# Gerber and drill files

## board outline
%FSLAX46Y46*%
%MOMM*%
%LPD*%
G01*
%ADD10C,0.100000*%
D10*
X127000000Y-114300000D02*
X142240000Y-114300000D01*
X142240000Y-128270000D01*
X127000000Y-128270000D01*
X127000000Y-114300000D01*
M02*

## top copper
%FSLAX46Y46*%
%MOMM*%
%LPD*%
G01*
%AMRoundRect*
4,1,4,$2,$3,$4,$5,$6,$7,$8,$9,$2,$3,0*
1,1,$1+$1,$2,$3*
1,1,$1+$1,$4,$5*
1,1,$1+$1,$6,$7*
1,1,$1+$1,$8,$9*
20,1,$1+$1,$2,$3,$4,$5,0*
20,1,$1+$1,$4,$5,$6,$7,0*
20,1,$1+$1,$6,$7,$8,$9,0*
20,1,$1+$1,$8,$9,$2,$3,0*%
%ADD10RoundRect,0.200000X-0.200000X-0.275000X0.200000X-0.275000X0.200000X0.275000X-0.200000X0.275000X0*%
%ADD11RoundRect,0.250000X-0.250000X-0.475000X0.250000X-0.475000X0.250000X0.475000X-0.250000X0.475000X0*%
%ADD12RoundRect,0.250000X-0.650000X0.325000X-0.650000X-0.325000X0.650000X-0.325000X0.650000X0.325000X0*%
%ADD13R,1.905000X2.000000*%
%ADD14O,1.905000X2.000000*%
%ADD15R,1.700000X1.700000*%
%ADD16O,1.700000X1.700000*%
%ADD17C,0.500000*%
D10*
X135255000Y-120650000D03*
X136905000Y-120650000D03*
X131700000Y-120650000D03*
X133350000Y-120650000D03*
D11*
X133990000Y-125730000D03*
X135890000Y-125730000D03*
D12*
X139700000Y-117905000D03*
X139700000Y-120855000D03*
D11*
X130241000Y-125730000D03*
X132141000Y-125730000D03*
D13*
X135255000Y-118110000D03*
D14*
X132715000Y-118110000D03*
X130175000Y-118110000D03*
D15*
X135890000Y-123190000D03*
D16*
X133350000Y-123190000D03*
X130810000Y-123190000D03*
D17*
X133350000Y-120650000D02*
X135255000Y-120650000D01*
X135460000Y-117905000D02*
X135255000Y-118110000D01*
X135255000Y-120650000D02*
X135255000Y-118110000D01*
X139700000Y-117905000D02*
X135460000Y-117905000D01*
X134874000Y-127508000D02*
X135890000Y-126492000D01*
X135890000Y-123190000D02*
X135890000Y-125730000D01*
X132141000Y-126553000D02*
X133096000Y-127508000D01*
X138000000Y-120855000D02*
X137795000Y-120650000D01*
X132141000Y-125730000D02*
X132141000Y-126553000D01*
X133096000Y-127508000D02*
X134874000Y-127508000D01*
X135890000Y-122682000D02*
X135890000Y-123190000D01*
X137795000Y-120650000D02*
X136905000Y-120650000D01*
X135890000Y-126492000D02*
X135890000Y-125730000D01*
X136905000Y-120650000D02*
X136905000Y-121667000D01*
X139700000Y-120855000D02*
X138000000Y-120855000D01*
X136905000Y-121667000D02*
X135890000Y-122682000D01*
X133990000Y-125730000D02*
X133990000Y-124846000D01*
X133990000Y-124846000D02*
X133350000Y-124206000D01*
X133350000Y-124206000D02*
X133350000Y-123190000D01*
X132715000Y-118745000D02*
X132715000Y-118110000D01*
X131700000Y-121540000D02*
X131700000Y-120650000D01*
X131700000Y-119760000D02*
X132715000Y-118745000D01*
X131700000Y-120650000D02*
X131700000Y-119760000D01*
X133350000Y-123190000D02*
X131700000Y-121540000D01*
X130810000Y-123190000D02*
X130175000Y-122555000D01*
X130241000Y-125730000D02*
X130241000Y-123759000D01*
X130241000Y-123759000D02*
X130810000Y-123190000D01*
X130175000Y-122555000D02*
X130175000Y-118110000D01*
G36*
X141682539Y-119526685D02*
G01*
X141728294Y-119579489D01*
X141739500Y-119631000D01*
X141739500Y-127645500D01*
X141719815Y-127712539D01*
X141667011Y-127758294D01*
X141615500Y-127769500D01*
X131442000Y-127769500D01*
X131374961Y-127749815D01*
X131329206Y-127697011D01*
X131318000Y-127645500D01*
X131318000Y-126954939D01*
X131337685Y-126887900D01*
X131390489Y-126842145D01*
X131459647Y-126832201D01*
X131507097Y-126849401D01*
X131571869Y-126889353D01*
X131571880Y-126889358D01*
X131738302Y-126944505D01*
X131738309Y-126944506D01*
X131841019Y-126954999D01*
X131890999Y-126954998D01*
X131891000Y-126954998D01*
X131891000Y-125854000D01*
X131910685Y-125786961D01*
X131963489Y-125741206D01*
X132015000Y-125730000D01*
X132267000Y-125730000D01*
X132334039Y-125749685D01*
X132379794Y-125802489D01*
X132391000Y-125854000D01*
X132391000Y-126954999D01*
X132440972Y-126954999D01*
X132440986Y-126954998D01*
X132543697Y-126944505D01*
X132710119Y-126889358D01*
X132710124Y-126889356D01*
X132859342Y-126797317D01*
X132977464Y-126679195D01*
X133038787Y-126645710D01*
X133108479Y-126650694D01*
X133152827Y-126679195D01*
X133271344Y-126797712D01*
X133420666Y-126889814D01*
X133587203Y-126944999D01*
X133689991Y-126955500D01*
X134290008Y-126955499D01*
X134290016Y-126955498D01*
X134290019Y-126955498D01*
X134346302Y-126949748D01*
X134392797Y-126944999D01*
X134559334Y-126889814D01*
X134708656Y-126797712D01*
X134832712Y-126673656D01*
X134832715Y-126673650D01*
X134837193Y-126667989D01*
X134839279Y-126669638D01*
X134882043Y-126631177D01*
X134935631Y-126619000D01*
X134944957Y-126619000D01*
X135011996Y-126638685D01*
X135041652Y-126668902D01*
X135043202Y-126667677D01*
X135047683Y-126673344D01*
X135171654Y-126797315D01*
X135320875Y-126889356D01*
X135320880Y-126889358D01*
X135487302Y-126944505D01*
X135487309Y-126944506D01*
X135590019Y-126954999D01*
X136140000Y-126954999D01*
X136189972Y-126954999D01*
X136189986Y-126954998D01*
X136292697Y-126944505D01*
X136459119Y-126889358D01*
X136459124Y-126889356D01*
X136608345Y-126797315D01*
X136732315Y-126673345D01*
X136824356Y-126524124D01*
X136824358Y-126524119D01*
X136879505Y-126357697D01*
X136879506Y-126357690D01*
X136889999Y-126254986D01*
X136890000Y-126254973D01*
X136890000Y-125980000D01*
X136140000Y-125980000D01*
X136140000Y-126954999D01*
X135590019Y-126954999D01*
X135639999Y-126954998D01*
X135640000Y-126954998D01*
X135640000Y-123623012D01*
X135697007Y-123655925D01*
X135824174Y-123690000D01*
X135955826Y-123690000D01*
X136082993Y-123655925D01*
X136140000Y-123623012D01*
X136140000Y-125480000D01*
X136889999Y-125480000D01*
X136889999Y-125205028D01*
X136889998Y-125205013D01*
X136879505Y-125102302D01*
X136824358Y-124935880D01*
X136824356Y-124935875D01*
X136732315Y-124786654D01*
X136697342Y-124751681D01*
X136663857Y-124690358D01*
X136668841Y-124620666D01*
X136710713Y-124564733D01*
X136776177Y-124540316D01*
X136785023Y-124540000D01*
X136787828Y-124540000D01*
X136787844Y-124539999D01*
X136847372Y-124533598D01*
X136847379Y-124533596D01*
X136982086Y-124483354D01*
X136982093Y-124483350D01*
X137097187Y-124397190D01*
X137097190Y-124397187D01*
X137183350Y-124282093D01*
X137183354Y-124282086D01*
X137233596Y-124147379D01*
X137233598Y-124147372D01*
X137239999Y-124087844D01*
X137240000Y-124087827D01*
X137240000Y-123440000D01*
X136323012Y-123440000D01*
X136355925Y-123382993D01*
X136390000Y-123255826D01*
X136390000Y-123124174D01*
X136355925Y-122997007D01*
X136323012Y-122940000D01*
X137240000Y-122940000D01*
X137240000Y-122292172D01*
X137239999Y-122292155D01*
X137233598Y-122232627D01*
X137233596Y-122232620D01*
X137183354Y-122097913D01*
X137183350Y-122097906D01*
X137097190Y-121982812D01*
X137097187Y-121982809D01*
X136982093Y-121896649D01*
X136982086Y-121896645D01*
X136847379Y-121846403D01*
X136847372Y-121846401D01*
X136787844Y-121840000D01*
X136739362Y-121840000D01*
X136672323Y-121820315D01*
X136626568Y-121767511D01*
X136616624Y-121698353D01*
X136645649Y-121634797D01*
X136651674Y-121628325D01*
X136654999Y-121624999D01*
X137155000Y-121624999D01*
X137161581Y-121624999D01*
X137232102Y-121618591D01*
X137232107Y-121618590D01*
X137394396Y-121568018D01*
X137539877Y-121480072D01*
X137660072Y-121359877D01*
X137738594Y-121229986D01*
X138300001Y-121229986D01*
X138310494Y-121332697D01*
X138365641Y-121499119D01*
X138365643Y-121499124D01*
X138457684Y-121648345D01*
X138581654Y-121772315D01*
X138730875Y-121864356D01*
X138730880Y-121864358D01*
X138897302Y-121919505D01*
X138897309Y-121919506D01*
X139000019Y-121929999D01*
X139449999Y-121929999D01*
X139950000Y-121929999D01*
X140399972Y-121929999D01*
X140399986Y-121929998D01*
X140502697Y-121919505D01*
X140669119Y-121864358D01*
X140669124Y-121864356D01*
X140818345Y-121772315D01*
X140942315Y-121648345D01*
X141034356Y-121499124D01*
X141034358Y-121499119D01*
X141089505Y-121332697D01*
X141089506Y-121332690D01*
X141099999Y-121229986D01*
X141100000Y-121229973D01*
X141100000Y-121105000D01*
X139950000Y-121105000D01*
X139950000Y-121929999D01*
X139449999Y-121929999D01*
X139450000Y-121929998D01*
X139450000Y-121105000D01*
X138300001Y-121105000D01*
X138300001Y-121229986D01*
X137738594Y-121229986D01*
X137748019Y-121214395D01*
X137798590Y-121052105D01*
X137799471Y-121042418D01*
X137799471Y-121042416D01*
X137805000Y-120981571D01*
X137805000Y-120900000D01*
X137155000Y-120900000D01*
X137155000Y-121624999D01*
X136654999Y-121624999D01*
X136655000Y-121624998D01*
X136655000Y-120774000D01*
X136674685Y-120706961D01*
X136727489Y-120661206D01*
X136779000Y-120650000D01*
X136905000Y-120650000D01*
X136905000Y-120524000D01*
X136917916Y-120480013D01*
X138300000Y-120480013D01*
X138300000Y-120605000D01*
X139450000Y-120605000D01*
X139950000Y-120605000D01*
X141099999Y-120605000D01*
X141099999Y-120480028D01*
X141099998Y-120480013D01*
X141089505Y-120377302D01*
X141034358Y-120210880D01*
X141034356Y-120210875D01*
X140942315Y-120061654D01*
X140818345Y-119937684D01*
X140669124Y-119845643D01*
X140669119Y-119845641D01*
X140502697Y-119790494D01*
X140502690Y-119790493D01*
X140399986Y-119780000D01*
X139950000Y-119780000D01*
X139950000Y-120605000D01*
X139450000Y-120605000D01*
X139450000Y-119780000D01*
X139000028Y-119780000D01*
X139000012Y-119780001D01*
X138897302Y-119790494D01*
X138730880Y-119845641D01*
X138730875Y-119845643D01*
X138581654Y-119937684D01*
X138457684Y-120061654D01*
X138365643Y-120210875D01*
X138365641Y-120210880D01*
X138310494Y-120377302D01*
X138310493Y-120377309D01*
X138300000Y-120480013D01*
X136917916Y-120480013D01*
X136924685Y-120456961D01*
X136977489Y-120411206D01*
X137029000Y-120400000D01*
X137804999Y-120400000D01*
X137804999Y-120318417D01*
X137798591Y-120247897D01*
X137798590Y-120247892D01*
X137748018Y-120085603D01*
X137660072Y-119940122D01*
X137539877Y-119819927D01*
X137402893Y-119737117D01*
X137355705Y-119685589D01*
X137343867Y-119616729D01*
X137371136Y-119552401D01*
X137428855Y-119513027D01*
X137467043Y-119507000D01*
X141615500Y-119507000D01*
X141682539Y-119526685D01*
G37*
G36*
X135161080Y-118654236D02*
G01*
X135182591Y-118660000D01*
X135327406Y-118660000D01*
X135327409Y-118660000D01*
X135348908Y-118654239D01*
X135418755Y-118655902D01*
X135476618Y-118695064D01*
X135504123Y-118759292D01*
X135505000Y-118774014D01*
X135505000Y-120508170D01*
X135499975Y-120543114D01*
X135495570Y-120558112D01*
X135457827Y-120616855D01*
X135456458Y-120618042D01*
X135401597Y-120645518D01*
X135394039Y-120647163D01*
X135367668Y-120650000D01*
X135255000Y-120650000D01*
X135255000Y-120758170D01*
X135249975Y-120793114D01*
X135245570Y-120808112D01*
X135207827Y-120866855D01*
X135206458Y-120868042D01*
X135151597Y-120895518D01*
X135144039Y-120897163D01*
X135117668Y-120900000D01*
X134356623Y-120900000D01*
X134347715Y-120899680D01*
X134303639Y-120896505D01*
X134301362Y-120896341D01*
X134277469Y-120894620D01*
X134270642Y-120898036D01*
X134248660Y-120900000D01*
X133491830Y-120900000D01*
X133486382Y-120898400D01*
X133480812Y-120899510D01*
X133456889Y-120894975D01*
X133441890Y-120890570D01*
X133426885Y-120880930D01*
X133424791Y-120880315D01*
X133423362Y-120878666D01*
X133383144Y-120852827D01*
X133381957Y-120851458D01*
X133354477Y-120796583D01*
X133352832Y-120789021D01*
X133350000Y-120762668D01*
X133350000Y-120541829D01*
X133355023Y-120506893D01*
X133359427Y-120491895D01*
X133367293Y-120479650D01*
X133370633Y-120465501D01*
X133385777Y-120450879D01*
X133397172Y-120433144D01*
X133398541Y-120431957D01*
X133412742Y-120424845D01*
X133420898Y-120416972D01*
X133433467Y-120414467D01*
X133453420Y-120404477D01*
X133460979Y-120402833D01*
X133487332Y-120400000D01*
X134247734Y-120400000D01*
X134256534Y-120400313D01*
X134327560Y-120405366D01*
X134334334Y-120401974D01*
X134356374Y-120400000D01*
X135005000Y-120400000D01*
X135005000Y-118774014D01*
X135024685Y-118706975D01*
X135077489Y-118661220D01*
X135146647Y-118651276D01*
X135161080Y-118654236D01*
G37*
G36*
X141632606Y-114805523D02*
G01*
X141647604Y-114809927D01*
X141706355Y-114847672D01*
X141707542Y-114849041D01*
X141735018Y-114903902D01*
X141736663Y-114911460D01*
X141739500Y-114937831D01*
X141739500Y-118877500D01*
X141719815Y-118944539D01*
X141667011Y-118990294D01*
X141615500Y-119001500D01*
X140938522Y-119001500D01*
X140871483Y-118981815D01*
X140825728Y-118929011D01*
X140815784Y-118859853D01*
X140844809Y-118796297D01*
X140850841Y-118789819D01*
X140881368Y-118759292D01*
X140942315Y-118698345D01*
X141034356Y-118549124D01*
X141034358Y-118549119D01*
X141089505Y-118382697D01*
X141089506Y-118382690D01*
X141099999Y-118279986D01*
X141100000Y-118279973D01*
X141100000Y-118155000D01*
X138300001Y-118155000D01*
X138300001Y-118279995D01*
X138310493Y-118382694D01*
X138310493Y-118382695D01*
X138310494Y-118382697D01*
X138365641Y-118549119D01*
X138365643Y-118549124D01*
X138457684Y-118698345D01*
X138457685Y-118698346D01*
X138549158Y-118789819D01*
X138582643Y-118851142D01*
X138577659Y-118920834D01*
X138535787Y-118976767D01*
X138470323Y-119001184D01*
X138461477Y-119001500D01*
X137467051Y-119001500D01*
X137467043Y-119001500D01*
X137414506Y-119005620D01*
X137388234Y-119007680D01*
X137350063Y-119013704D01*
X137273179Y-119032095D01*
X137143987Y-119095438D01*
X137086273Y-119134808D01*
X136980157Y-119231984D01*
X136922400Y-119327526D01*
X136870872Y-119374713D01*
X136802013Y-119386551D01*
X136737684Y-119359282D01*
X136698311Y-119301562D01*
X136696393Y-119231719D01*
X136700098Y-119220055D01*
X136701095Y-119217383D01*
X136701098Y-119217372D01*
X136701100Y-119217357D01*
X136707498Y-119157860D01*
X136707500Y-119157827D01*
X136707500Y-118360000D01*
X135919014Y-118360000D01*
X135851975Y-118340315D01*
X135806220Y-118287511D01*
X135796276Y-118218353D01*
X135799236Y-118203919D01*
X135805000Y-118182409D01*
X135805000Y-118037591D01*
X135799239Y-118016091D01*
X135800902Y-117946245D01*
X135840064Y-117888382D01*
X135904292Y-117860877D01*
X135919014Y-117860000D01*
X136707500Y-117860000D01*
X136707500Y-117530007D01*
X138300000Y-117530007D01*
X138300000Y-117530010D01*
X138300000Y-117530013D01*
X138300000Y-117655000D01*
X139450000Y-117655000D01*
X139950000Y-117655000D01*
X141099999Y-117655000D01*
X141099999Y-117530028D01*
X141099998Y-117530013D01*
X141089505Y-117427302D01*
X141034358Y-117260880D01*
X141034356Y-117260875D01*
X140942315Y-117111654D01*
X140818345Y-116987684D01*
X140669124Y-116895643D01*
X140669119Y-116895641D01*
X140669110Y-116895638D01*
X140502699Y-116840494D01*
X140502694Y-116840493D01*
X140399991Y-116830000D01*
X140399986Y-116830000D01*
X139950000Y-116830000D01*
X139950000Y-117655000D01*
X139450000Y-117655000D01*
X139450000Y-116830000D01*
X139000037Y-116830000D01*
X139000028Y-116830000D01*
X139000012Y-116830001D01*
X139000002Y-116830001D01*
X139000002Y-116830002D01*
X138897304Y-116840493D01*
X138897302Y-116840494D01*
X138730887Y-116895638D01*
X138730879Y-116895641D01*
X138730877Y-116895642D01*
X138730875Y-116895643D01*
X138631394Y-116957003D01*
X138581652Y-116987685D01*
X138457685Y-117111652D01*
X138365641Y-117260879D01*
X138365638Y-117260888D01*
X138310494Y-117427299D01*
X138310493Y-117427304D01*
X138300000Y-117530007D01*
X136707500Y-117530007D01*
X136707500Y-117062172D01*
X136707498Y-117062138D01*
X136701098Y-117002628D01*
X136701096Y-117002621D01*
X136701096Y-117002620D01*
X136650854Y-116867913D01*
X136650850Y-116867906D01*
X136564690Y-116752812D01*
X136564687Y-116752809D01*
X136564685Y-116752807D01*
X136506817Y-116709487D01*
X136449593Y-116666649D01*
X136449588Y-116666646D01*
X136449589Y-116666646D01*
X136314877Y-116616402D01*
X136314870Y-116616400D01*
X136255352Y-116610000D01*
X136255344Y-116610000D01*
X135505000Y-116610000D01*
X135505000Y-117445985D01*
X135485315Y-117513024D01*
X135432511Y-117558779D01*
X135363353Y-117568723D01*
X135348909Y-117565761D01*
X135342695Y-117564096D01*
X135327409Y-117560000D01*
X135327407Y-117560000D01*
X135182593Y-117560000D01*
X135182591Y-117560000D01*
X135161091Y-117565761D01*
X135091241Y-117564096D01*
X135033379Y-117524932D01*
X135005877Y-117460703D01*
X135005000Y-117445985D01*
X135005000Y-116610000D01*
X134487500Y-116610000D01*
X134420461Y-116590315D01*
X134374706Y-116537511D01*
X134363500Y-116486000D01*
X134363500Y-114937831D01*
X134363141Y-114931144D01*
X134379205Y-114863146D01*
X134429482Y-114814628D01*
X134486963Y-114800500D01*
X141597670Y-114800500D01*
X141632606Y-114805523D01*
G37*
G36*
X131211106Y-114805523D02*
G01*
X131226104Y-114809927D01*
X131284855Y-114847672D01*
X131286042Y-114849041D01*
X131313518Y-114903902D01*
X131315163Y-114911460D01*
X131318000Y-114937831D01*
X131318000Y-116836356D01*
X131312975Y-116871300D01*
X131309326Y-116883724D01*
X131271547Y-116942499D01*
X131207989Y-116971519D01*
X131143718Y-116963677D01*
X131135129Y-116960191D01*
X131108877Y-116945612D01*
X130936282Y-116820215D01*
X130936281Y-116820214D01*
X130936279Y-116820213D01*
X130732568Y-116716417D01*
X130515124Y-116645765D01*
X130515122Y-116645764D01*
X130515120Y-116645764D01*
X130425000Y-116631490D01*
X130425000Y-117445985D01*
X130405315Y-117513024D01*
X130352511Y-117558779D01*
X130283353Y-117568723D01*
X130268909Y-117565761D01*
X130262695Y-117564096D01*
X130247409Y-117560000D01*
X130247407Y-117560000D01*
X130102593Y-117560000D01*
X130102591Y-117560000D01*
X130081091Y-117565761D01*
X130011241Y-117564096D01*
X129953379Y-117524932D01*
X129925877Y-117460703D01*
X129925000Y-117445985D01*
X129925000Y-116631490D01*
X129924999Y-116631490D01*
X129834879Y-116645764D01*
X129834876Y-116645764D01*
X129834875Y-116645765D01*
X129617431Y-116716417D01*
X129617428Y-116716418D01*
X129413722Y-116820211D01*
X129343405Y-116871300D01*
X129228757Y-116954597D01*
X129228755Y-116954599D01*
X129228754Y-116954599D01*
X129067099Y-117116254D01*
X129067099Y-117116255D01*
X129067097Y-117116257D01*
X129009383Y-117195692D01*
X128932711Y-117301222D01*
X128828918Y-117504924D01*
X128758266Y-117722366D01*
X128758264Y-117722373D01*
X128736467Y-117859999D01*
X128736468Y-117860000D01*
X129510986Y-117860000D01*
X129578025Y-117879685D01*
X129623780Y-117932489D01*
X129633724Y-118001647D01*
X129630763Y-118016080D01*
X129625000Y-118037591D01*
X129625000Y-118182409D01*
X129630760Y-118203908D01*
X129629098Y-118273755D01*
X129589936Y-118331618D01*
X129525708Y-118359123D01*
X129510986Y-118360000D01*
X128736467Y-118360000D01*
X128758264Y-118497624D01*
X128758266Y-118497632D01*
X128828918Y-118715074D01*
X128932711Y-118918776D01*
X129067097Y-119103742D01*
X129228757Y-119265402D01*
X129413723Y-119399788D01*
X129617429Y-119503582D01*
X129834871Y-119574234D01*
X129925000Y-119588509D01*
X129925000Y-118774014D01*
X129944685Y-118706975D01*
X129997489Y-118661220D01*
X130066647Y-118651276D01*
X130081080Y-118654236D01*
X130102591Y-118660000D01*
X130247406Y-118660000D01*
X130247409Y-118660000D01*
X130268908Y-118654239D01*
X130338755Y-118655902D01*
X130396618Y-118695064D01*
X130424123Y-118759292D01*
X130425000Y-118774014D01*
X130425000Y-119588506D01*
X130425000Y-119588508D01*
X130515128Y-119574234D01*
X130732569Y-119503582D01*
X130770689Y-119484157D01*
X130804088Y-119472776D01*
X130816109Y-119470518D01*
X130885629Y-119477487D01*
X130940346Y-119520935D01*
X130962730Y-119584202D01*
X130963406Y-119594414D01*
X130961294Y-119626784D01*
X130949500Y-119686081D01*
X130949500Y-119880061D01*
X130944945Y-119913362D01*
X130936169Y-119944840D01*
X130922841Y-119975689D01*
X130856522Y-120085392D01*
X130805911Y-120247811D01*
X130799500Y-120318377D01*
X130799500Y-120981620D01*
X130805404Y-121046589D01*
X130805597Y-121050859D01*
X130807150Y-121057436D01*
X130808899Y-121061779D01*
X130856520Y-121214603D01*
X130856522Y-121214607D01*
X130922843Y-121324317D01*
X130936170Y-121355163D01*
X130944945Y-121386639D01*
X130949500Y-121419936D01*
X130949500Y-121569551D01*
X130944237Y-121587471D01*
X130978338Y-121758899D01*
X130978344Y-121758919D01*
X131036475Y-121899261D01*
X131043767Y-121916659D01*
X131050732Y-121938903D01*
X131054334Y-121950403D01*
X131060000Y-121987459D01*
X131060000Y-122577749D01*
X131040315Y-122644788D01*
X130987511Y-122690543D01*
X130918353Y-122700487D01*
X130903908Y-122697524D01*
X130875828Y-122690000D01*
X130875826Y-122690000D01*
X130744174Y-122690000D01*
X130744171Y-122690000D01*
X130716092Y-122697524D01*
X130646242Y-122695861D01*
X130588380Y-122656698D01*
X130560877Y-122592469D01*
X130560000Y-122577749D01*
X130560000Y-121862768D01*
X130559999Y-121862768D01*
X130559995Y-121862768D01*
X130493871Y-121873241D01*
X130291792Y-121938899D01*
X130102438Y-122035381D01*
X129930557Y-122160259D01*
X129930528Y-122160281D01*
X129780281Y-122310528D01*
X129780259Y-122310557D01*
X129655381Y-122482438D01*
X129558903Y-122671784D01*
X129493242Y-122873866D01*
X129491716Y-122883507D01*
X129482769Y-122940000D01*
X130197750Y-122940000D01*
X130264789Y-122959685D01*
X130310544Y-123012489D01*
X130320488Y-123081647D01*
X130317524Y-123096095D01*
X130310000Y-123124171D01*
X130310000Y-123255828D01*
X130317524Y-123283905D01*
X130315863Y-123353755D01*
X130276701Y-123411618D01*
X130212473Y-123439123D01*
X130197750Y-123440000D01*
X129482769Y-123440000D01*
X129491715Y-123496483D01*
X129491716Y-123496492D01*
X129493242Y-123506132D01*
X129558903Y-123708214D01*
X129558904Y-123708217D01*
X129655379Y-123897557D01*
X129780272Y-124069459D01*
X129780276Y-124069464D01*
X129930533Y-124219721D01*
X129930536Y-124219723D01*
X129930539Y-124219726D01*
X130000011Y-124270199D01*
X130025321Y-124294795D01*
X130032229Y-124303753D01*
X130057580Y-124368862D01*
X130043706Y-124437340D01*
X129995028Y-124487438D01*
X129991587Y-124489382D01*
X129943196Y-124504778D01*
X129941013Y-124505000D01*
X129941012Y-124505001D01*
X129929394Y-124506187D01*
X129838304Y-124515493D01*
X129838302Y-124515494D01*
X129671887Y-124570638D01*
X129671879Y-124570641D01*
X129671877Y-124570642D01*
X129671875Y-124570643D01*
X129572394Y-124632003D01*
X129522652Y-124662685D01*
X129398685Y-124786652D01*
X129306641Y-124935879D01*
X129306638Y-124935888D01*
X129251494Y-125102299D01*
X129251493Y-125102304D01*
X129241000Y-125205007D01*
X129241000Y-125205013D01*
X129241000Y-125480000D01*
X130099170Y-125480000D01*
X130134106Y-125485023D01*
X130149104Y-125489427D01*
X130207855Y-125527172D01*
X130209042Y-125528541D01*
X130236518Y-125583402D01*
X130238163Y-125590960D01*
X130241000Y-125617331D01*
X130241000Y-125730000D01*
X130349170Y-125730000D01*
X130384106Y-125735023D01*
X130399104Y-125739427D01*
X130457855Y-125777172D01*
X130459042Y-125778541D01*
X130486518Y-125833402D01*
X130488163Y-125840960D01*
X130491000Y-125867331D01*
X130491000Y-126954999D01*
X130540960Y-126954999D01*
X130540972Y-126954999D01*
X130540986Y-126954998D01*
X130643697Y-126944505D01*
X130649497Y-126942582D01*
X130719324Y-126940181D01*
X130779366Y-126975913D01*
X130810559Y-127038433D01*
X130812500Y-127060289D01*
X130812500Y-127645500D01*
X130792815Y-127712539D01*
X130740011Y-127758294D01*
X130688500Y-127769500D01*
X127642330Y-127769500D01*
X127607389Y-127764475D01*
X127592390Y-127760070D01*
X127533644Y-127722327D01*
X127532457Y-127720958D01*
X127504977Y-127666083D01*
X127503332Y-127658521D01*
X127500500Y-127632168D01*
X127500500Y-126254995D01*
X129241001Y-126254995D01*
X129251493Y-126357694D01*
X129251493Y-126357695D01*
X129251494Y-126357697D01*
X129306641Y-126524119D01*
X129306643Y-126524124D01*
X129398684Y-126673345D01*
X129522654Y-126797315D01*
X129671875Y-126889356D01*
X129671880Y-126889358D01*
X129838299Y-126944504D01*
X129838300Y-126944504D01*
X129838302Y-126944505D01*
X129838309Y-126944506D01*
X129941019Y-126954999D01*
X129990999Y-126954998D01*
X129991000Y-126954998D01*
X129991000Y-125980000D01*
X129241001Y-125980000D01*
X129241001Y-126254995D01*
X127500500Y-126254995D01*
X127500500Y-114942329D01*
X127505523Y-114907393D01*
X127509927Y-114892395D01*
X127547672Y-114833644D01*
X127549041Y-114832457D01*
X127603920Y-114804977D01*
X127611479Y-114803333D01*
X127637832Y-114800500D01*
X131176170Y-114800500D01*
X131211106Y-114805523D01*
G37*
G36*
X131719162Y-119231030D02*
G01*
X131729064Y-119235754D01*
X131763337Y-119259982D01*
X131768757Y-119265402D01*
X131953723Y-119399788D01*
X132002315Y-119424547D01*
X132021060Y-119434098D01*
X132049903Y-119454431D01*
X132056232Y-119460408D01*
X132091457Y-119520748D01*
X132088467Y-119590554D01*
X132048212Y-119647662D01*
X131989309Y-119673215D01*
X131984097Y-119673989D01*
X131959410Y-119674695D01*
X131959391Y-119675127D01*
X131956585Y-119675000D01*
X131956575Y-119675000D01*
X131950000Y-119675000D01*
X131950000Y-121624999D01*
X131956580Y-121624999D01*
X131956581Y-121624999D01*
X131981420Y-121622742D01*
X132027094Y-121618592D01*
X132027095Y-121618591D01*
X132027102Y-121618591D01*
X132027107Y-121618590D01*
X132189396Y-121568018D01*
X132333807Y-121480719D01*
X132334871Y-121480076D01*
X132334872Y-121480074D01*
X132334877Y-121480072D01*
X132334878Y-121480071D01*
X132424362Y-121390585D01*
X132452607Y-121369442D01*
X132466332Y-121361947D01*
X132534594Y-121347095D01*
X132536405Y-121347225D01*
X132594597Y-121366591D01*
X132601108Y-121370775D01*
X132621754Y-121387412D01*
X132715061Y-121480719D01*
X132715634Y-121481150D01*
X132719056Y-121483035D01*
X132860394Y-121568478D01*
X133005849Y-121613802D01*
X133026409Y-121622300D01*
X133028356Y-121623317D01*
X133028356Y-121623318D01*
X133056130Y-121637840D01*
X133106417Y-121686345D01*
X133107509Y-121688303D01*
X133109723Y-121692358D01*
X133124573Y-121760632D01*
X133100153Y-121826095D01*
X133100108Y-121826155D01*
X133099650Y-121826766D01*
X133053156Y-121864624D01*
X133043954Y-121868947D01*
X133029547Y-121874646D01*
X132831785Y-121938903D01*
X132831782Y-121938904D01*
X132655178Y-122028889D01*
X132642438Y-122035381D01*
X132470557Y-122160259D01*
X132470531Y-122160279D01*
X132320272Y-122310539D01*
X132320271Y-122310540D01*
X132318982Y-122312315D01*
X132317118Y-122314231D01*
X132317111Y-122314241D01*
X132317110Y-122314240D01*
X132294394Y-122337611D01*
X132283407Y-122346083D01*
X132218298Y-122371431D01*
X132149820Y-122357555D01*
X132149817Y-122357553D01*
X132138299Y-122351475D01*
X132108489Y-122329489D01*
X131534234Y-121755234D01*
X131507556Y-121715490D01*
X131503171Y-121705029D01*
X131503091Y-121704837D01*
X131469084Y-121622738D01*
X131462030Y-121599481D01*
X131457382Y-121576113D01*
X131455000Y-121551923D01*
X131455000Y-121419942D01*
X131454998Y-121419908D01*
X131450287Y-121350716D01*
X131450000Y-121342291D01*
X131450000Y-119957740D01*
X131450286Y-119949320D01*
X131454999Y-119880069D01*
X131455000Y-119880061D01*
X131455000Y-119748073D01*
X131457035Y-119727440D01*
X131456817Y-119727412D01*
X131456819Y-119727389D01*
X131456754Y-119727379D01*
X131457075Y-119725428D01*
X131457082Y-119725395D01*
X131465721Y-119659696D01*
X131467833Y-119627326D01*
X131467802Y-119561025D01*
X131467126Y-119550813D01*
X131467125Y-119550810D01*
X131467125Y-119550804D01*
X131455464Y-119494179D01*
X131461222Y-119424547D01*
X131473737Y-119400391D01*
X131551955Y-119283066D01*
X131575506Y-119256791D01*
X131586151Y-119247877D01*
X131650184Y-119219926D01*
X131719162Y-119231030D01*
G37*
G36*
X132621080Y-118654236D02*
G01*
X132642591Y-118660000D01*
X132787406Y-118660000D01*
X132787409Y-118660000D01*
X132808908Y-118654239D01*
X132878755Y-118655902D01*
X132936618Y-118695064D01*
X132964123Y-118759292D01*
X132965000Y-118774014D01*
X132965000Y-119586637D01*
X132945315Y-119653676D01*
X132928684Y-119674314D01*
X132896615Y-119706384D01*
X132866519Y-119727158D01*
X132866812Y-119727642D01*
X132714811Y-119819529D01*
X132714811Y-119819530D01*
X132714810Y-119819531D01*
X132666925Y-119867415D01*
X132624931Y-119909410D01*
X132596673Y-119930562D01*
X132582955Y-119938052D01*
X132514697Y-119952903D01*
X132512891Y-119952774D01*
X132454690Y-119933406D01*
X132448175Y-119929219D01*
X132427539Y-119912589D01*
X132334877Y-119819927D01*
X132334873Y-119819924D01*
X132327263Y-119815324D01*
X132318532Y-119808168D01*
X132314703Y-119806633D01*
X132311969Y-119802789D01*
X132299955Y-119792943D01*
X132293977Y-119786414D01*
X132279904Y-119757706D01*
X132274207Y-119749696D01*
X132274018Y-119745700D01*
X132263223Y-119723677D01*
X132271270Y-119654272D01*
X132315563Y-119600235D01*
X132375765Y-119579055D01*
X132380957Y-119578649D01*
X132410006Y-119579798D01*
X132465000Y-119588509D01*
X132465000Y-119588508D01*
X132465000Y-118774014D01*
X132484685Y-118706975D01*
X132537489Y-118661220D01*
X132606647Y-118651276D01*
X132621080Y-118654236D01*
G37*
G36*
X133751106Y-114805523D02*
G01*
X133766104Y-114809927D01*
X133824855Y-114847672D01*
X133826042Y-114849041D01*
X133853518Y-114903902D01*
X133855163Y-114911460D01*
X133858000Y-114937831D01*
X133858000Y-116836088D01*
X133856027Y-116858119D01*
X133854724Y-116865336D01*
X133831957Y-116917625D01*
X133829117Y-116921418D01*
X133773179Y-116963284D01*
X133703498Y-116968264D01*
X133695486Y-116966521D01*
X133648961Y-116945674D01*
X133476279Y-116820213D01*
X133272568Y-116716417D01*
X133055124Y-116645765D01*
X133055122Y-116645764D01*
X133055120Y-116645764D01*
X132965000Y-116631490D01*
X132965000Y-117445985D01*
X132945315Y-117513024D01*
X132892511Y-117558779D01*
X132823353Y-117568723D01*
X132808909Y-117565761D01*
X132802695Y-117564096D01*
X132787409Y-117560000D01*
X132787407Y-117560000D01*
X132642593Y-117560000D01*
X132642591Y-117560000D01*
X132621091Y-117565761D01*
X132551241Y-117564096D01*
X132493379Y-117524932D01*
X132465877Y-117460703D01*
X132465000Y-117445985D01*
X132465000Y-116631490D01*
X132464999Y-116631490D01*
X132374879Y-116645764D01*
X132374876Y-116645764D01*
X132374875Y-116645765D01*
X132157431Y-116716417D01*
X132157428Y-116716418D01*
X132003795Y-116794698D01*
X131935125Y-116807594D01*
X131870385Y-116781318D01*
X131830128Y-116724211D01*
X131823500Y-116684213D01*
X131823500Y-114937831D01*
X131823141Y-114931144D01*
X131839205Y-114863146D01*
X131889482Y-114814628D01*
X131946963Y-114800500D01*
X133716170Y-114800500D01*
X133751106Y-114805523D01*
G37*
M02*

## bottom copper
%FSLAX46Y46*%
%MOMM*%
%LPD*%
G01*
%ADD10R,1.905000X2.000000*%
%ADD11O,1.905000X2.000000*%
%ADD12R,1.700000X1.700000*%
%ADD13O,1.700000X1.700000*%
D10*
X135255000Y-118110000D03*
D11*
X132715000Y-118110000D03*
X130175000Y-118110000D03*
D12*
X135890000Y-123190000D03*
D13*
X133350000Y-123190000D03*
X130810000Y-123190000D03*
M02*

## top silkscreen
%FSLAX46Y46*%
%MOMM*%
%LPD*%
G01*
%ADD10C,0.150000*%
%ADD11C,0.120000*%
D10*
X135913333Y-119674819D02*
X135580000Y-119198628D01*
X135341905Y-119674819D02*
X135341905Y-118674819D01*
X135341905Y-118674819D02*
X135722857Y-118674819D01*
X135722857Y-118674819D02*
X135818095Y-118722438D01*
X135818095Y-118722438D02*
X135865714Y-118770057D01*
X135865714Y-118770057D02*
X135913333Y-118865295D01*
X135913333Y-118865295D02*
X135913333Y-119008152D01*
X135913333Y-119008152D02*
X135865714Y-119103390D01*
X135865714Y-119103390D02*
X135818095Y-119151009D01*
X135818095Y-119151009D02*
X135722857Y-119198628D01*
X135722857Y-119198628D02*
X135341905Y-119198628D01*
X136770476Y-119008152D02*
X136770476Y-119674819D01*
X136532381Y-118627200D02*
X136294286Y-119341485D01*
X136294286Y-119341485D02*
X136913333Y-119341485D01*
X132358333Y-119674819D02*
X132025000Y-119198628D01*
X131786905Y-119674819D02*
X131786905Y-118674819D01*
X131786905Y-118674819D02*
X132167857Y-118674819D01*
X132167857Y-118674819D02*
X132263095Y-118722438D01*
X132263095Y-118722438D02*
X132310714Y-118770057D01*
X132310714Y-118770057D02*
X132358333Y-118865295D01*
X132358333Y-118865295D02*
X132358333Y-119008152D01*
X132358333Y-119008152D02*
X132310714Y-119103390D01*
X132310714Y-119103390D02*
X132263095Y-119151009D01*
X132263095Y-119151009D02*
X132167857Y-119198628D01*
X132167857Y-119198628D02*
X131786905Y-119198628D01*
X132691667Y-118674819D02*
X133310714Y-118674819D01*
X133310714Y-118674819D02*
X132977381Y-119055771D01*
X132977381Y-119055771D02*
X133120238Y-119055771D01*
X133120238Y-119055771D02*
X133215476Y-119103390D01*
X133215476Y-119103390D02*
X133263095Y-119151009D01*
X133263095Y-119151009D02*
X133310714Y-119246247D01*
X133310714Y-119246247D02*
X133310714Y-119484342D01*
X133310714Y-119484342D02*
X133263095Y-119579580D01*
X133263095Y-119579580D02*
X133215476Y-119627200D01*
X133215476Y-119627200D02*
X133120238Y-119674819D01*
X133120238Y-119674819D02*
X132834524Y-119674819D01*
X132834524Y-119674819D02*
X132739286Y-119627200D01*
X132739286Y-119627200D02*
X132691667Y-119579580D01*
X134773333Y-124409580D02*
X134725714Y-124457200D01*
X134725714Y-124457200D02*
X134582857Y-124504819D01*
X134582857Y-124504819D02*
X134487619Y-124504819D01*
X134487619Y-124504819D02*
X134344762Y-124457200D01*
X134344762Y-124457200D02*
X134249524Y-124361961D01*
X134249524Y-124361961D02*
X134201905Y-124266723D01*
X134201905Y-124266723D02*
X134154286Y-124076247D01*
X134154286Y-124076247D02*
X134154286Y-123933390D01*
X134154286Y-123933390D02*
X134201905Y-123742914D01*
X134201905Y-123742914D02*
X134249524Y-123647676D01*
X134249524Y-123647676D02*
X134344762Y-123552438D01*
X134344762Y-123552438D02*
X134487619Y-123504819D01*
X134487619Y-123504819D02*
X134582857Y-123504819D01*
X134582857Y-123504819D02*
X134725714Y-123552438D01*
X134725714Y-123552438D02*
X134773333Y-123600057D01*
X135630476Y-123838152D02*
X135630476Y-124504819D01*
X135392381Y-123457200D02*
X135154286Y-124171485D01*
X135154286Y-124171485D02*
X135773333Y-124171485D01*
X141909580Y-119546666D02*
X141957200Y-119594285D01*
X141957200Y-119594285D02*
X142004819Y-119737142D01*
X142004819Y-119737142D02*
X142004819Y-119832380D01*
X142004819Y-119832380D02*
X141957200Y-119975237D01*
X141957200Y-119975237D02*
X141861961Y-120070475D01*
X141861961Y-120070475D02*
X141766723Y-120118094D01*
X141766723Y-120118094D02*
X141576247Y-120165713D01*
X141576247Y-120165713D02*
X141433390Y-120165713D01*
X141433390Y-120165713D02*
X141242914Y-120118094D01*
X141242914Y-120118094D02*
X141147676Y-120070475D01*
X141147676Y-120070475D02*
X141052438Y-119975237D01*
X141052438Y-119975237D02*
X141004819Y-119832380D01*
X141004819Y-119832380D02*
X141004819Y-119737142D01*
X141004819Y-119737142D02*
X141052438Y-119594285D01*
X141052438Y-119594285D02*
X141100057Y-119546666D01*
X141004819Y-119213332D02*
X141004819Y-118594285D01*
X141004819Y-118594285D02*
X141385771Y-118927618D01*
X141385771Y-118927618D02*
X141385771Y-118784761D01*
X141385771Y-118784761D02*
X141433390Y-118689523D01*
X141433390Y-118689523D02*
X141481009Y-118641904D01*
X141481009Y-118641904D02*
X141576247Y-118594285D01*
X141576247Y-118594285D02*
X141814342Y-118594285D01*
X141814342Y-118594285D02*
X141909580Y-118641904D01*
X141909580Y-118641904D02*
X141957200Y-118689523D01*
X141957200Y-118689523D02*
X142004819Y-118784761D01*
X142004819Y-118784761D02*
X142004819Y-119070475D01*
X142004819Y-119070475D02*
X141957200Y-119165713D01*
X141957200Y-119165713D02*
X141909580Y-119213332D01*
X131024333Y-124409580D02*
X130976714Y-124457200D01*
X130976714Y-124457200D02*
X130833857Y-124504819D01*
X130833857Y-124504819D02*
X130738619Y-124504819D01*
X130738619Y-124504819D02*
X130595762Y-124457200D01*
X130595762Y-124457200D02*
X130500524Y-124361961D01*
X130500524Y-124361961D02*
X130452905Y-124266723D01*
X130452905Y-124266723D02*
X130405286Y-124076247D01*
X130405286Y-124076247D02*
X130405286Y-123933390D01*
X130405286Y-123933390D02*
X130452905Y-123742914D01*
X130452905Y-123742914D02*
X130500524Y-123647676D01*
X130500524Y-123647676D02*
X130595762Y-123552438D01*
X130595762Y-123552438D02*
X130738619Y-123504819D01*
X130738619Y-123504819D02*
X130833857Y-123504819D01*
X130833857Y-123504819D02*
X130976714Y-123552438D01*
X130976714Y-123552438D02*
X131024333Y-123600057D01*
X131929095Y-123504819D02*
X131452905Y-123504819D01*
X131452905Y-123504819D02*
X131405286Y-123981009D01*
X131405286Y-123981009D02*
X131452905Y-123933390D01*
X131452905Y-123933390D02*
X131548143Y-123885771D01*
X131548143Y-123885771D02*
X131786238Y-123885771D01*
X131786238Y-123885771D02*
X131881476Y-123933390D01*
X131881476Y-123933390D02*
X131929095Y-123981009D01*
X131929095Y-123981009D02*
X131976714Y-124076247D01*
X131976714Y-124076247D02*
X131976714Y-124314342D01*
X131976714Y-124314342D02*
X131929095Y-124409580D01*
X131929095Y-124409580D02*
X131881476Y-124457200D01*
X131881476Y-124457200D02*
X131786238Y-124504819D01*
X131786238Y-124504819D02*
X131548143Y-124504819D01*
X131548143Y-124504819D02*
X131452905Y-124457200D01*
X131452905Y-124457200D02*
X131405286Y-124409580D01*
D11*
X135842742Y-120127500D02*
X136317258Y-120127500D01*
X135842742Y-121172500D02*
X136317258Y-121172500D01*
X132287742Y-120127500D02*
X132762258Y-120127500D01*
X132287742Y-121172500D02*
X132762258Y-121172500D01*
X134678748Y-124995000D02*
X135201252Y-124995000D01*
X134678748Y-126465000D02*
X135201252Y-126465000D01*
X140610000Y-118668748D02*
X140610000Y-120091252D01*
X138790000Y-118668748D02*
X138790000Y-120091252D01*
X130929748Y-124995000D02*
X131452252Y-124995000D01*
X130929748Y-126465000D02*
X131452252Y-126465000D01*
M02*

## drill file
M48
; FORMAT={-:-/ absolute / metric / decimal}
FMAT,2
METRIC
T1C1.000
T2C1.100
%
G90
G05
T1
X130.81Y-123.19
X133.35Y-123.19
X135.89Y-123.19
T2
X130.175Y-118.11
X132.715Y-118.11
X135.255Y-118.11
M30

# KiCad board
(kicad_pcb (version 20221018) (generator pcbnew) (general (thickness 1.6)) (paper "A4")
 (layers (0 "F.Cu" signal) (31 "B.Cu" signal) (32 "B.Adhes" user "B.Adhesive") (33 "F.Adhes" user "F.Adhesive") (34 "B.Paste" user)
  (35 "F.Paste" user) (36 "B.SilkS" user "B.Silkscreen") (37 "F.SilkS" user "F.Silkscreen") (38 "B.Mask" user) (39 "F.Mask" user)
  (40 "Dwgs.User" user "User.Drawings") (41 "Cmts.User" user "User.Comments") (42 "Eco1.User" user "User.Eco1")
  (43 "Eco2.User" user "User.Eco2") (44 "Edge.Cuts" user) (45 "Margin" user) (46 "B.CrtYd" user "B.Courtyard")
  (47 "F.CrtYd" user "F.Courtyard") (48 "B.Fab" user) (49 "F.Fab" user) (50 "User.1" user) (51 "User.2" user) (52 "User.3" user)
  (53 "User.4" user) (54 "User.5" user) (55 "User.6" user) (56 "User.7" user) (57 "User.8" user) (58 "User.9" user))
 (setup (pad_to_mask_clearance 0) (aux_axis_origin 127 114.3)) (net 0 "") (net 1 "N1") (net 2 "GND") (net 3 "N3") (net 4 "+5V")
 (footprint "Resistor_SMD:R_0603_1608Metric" (layer "F.Cu") (at 136.08 120.65)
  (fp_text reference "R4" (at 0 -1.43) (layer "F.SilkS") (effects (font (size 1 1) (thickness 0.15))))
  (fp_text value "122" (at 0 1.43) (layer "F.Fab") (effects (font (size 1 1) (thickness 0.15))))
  (fp_line (start -0.237258 -0.5225) (end 0.237258 -0.5225) (stroke (width 0.12) (type solid)) (layer "F.SilkS"))
  (fp_line (start -0.237258 0.5225) (end 0.237258 0.5225) (stroke (width 0.12) (type solid)) (layer "F.SilkS"))
  (pad "1" smd roundrect (at -0.825 0) (size 0.8 0.95) (layers "F.Cu" "F.Paste" "F.Mask") (roundrect_rratio 0.25) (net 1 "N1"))
  (pad "2" smd roundrect (at 0.825 0) (size 0.8 0.95) (layers "F.Cu" "F.Paste" "F.Mask") (roundrect_rratio 0.25) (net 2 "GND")))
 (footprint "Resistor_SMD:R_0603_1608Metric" (layer "F.Cu") (at 132.525 120.65)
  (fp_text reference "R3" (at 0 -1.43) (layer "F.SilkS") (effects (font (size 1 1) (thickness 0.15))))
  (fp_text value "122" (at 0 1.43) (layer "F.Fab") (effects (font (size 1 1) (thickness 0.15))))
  (fp_line (start -0.237258 -0.5225) (end 0.237258 -0.5225) (stroke (width 0.12) (type solid)) (layer "F.SilkS"))
  (fp_line (start -0.237258 0.5225) (end 0.237258 0.5225) (stroke (width 0.12) (type solid)) (layer "F.SilkS"))
  (pad "1" smd roundrect (at -0.825 0) (size 0.8 0.95) (layers "F.Cu" "F.Paste" "F.Mask") (roundrect_rratio 0.25) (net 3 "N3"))
  (pad "2" smd roundrect (at 0.825 0) (size 0.8 0.95) (layers "F.Cu" "F.Paste" "F.Mask") (roundrect_rratio 0.25) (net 1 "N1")))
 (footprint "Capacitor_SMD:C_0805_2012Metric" (layer "F.Cu") (at 134.94 125.73)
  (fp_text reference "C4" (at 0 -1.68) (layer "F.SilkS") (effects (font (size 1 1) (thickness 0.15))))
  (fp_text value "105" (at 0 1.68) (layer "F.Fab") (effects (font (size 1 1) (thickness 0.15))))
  (fp_line (start -0.261252 -0.735) (end 0.261252 -0.735) (stroke (width 0.12) (type solid)) (layer "F.SilkS"))
  (fp_line (start -0.261252 0.735) (end 0.261252 0.735) (stroke (width 0.12) (type solid)) (layer "F.SilkS"))
  (pad "1" smd roundrect (at -0.95 0) (size 1 1.45) (layers "F.Cu" "F.Paste" "F.Mask") (roundrect_rratio 0.25) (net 3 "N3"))
  (pad "2" smd roundrect (at 0.95 0) (size 1 1.45) (layers "F.Cu" "F.Paste" "F.Mask") (roundrect_rratio 0.25) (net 2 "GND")))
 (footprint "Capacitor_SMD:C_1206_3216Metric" (layer "F.Cu") (at 139.7 119.38 -90)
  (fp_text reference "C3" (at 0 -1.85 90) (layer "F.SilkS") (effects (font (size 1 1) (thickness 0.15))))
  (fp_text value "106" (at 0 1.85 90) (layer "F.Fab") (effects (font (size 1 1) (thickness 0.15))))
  (fp_line (start -0.711252 -0.91) (end 0.711252 -0.91) (stroke (width 0.12) (type solid)) (layer "F.SilkS"))
  (fp_line (start -0.711252 0.91) (end 0.711252 0.91) (stroke (width 0.12) (type solid)) (layer "F.SilkS"))
  (pad "1" smd roundrect (at -1.475 0 270) (size 1.15 1.8) (layers "F.Cu" "F.Paste" "F.Mask") (roundrect_rratio 0.2173913043) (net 1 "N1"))
  (pad "2" smd roundrect (at 1.475 0 270) (size 1.15 1.8) (layers "F.Cu" "F.Paste" "F.Mask") (roundrect_rratio 0.2173913043) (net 2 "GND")))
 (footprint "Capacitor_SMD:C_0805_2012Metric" (layer "F.Cu") (at 131.191 125.73)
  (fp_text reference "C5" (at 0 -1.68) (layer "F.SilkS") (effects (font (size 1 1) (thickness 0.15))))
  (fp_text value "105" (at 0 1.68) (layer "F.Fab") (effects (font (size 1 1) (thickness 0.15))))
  (fp_line (start -0.261252 -0.735) (end 0.261252 -0.735) (stroke (width 0.12) (type solid)) (layer "F.SilkS"))
  (fp_line (start -0.261252 0.735) (end 0.261252 0.735) (stroke (width 0.12) (type solid)) (layer "F.SilkS"))
  (pad "1" smd roundrect (at -0.95 0) (size 1 1.45) (layers "F.Cu" "F.Paste" "F.Mask") (roundrect_rratio 0.25) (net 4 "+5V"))
  (pad "2" smd roundrect (at 0.95 0) (size 1 1.45) (layers "F.Cu" "F.Paste" "F.Mask") (roundrect_rratio 0.25) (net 2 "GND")))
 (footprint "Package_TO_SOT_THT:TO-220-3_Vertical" (layer "B.Cu") (at 135.255 118.11 180)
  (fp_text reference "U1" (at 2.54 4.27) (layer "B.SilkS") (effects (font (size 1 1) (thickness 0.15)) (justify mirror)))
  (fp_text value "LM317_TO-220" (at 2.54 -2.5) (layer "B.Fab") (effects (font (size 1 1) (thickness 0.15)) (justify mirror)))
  (pad "1" thru_hole rect (at 0 0 180) (size 1.905 2) (drill 1.1) (layers "*.Cu" "*.Mask") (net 1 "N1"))
  (pad "2" thru_hole oval (at 2.54 0 180) (size 1.905 2) (drill 1.1) (layers "*.Cu" "*.Mask") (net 3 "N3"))
  (pad "3" thru_hole oval (at 5.08 0 180) (size 1.905 2) (drill 1.1) (layers "*.Cu" "*.Mask") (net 4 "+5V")))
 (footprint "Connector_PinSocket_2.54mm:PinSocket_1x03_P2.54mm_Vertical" (layer "B.Cu") (at 135.89 123.19 90)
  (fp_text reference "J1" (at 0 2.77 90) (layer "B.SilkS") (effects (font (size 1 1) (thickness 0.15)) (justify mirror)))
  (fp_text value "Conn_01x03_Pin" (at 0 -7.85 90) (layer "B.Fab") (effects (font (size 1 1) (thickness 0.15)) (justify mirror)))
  (pad "1" thru_hole rect (at 0 0 90) (size 1.7 1.7) (drill 1) (layers "*.Cu" "*.Mask") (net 2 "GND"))
  (pad "2" thru_hole oval (at 0 -2.54 90) (size 1.7 1.7) (drill 1) (layers "*.Cu" "*.Mask") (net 3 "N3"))
  (pad "3" thru_hole oval (at 0 -5.08 90) (size 1.7 1.7) (drill 1) (layers "*.Cu" "*.Mask") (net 4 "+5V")))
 (gr_rect (start 127 114.3) (end 142.24 128.27) (stroke (width 0.1) (type default)) (fill none) (layer "Edge.Cuts"))
 (segment (start 133.35 120.65) (end 135.255 120.65) (width 0.5) (layer "F.Cu") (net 1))
 (segment (start 135.46 117.905) (end 135.255 118.11) (width 0.5) (layer "F.Cu") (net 1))
 (segment (start 135.255 120.65) (end 135.255 118.11) (width 0.5) (layer "F.Cu") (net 1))
 (segment (start 139.7 117.905) (end 135.46 117.905) (width 0.5) (layer "F.Cu") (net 1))
 (segment (start 134.874 127.508) (end 135.89 126.492) (width 0.5) (layer "F.Cu") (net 2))
 (segment (start 135.89 123.19) (end 135.89 125.73) (width 0.5) (layer "F.Cu") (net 2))
 (segment (start 132.141 126.553) (end 133.096 127.508) (width 0.5) (layer "F.Cu") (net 2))
 (segment (start 138 120.855) (end 137.795 120.65) (width 0.5) (layer "F.Cu") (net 2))
 (segment (start 132.141 125.73) (end 132.141 126.553) (width 0.5) (layer "F.Cu") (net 2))
 (segment (start 133.096 127.508) (end 134.874 127.508) (width 0.5) (layer "F.Cu") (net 2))
 (segment (start 135.89 122.682) (end 135.89 123.19) (width 0.5) (layer "F.Cu") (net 2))
 (segment (start 137.795 120.65) (end 136.905 120.65) (width 0.5) (layer "F.Cu") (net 2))
 (segment (start 135.89 126.492) (end 135.89 125.73) (width 0.5) (layer "F.Cu") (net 2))
 (segment (start 136.905 120.65) (end 136.905 121.667) (width 0.5) (layer "F.Cu") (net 2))
 (segment (start 139.7 120.855) (end 138 120.855) (width 0.5) (layer "F.Cu") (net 2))
 (segment (start 136.905 121.667) (end 135.89 122.682) (width 0.5) (layer "F.Cu") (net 2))
 (segment (start 133.99 125.73) (end 133.99 124.846) (width 0.5) (layer "F.Cu") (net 3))
 (segment (start 133.99 124.846) (end 133.35 124.206) (width 0.5) (layer "F.Cu") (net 3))
 (segment (start 133.35 124.206) (end 133.35 123.19) (width 0.5) (layer "F.Cu") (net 3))
 (segment (start 132.715 118.745) (end 132.715 118.11) (width 0.5) (layer "F.Cu") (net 3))
 (segment (start 131.7 121.54) (end 131.7 120.65) (width 0.5) (layer "F.Cu") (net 3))
 (segment (start 131.7 119.76) (end 132.715 118.745) (width 0.5) (layer "F.Cu") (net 3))
 (segment (start 131.7 120.65) (end 131.7 119.76) (width 0.5) (layer "F.Cu") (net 3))
 (segment (start 133.35 123.19) (end 131.7 121.54) (width 0.5) (layer "F.Cu") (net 3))
 (segment (start 130.81 123.19) (end 130.175 122.555) (width 0.5) (layer "F.Cu") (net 4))
 (segment (start 130.241 125.73) (end 130.241 123.759) (width 0.5) (layer "F.Cu") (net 4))
 (segment (start 130.241 123.759) (end 130.81 123.19) (width 0.5) (layer "F.Cu") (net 4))
 (segment (start 130.175 122.555) (end 130.175 118.11) (width 0.5) (layer "F.Cu") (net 4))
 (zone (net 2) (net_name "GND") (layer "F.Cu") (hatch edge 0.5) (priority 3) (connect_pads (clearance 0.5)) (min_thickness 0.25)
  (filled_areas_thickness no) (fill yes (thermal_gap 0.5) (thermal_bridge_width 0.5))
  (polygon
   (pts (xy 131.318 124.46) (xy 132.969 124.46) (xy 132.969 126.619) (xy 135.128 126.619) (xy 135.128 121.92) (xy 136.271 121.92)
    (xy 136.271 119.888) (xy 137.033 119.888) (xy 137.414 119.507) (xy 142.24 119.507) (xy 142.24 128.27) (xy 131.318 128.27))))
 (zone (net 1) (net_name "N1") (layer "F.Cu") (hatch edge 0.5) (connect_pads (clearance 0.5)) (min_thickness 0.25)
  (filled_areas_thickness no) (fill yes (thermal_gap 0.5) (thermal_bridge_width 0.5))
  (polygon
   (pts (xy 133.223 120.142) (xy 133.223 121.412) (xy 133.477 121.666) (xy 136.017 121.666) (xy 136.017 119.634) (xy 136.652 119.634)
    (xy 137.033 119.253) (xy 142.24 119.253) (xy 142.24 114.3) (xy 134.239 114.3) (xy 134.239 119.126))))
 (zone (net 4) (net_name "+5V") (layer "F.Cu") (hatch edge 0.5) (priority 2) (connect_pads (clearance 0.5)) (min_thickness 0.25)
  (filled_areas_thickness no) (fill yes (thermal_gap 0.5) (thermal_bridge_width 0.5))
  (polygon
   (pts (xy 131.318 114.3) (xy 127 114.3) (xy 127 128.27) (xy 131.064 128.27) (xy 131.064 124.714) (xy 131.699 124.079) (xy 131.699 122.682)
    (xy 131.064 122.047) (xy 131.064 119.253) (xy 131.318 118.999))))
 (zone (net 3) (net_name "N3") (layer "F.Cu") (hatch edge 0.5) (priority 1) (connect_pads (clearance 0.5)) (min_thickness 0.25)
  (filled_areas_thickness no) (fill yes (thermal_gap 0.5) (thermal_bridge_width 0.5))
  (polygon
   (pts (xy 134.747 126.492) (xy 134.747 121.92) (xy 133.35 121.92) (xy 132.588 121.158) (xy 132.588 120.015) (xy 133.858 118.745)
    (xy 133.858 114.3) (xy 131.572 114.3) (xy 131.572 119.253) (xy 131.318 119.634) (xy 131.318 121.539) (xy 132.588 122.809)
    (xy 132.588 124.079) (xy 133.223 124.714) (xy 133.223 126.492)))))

